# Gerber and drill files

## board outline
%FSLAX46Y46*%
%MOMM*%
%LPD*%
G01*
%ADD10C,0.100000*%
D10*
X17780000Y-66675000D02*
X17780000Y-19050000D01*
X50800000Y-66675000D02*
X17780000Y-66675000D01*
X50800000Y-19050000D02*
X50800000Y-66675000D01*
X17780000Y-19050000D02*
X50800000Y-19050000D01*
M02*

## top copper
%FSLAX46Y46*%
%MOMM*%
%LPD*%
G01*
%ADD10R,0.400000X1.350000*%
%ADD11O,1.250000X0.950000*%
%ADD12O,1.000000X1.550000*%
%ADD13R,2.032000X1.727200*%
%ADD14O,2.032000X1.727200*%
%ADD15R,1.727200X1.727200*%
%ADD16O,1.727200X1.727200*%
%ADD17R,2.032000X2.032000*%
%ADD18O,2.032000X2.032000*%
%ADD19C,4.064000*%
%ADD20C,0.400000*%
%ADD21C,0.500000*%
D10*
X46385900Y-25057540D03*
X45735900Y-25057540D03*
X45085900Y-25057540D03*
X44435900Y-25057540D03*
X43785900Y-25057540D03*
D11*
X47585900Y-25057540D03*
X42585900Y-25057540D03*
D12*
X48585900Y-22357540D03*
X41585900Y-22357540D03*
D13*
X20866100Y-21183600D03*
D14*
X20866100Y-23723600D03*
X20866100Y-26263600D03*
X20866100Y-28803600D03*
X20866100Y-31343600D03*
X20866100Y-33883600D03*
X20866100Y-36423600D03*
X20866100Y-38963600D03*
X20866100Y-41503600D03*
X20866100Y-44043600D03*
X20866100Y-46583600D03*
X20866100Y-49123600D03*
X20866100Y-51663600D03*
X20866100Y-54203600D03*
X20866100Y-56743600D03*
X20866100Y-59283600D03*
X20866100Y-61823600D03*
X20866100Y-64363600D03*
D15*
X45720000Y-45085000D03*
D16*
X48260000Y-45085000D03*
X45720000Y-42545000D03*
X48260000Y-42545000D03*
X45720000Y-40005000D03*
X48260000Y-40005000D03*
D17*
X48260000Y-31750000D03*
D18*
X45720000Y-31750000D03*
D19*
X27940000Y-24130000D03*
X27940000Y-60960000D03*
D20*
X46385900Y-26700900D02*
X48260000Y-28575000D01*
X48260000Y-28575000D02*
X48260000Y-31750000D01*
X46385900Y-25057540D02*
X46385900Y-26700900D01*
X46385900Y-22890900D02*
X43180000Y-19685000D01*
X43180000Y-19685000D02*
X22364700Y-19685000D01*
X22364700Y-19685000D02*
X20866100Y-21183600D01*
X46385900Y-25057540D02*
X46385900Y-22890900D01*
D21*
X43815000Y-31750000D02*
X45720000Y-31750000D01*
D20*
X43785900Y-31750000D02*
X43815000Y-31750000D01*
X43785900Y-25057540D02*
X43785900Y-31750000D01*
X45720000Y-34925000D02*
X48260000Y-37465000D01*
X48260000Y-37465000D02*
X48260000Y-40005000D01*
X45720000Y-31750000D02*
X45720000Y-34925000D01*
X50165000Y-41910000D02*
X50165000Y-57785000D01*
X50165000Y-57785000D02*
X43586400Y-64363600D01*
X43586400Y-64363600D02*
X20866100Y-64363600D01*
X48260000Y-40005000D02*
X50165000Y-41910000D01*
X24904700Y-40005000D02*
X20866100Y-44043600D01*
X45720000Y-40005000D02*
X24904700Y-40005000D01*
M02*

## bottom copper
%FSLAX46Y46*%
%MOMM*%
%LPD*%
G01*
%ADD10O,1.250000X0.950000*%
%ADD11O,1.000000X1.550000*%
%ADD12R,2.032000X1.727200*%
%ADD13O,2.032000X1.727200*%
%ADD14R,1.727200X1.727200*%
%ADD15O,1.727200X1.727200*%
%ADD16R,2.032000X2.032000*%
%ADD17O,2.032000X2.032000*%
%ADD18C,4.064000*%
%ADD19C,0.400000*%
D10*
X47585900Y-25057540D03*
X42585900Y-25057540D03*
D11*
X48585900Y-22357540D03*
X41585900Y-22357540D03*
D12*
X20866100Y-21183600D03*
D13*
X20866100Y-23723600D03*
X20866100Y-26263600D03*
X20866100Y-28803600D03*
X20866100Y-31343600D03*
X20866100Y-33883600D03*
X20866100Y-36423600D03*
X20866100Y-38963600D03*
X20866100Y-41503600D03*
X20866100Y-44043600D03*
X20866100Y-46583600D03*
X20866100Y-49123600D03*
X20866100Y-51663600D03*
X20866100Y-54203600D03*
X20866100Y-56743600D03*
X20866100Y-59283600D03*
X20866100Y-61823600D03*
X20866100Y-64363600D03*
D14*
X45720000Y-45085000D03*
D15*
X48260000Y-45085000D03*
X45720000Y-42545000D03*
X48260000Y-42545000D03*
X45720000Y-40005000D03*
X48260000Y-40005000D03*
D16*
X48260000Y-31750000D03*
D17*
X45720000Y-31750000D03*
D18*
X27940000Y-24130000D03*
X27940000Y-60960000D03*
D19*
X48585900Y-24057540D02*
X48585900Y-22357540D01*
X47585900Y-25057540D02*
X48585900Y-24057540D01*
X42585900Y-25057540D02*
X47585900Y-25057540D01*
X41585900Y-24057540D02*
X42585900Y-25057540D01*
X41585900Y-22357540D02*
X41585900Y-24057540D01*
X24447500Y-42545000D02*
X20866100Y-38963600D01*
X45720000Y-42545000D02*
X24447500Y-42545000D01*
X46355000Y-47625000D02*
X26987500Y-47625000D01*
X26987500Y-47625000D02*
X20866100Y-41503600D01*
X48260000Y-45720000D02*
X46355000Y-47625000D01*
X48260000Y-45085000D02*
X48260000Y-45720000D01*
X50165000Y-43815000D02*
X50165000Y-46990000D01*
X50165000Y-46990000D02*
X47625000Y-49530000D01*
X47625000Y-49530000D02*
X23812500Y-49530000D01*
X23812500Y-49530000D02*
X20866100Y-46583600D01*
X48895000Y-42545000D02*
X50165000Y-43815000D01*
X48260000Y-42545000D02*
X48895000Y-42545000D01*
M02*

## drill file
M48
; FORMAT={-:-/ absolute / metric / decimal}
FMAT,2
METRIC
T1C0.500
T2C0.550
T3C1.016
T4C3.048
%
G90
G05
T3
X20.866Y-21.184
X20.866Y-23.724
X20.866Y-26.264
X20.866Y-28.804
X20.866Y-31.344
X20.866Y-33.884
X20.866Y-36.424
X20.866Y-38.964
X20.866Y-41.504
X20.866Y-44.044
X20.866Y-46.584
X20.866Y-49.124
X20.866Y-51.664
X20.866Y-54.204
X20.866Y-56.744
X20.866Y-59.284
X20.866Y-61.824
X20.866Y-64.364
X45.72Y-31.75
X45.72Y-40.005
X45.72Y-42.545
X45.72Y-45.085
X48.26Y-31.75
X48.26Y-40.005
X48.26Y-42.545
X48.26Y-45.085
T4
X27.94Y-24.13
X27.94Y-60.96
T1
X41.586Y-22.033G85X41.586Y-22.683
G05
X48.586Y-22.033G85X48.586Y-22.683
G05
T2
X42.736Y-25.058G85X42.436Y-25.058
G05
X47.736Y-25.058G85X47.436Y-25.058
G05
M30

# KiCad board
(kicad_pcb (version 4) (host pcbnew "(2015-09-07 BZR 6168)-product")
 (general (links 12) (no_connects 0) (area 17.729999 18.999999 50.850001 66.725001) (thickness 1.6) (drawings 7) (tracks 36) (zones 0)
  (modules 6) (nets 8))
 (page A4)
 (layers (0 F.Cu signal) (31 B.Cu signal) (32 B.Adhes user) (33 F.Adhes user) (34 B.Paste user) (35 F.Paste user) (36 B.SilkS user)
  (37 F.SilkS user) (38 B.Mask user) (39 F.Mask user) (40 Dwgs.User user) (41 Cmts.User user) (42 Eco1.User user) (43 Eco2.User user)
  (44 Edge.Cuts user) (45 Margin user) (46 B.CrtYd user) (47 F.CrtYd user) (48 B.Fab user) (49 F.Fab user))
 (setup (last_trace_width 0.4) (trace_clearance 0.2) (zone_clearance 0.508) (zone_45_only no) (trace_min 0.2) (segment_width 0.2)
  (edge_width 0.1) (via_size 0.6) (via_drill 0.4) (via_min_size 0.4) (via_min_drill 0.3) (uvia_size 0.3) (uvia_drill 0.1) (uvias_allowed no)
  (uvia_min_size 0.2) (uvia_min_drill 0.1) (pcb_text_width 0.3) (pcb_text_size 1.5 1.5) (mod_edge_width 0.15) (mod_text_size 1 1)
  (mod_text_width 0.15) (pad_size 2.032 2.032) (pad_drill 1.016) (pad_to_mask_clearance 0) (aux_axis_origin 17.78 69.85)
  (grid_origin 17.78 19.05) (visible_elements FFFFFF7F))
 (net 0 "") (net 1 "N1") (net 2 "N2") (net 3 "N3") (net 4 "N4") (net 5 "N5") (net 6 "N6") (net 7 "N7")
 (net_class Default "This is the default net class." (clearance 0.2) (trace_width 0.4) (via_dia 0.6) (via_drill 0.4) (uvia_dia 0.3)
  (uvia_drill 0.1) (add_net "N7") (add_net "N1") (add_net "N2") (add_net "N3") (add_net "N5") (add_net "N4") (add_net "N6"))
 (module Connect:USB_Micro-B (layer F.Cu) (at 45.085 23.495 180)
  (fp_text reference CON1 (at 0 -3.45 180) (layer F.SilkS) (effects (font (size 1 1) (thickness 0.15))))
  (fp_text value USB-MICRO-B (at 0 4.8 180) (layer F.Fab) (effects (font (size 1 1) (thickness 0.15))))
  (pad 1 smd rect (at -1.3009 -1.56254 270) (size 1.35 0.4) (layers F.Cu F.Paste F.Mask) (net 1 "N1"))
  (pad 2 smd rect (at -0.6509 -1.56254 270) (size 1.35 0.4) (layers F.Cu F.Paste F.Mask))
  (pad 3 smd rect (at -0.0009 -1.56254 270) (size 1.35 0.4) (layers F.Cu F.Paste F.Mask))
  (pad 4 smd rect (at 0.6491 -1.56254 270) (size 1.35 0.4) (layers F.Cu F.Paste F.Mask))
  (pad 5 smd rect (at 1.2991 -1.56254 270) (size 1.35 0.4) (layers F.Cu F.Paste F.Mask) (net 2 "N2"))
  (pad 6 thru_hole oval (at -2.5009 -1.56254 270) (size 0.95 1.25) (drill oval 0.55 0.85) (layers *.Cu *.Mask F.SilkS) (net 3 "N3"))
  (pad 6 thru_hole oval (at 2.4991 -1.56254 270) (size 0.95 1.25) (drill oval 0.55 0.85) (layers *.Cu *.Mask F.SilkS) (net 3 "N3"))
  (pad 6 thru_hole oval (at -3.5009 1.13746 270) (size 1.55 1) (drill oval 1.15 0.5) (layers *.Cu *.Mask F.SilkS) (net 3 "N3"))
  (pad 6 thru_hole oval (at 3.4991 1.13746 270) (size 1.55 1) (drill oval 1.15 0.5) (layers *.Cu *.Mask F.SilkS) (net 3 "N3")))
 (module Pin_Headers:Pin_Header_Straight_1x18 (layer F.Cu) (at 20.8661 21.1836)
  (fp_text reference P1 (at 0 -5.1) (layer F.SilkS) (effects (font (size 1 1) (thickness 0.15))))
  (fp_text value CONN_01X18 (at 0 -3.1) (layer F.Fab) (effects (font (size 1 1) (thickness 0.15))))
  (pad 1 thru_hole rect (at 0 0) (size 2.032 1.7272) (drill 1.016) (layers *.Cu *.Mask F.SilkS) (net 1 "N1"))
  (pad 2 thru_hole oval (at 0 2.54) (size 2.032 1.7272) (drill 1.016) (layers *.Cu *.Mask F.SilkS))
  (pad 3 thru_hole oval (at 0 5.08) (size 2.032 1.7272) (drill 1.016) (layers *.Cu *.Mask F.SilkS))
  (pad 4 thru_hole oval (at 0 7.62) (size 2.032 1.7272) (drill 1.016) (layers *.Cu *.Mask F.SilkS))
  (pad 5 thru_hole oval (at 0 10.16) (size 2.032 1.7272) (drill 1.016) (layers *.Cu *.Mask F.SilkS))
  (pad 6 thru_hole oval (at 0 12.7) (size 2.032 1.7272) (drill 1.016) (layers *.Cu *.Mask F.SilkS))
  (pad 7 thru_hole oval (at 0 15.24) (size 2.032 1.7272) (drill 1.016) (layers *.Cu *.Mask F.SilkS))
  (pad 8 thru_hole oval (at 0 17.78) (size 2.032 1.7272) (drill 1.016) (layers *.Cu *.Mask F.SilkS) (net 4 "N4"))
  (pad 9 thru_hole oval (at 0 20.32) (size 2.032 1.7272) (drill 1.016) (layers *.Cu *.Mask F.SilkS) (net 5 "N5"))
  (pad 10 thru_hole oval (at 0 22.86) (size 2.032 1.7272) (drill 1.016) (layers *.Cu *.Mask F.SilkS) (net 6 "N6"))
  (pad 11 thru_hole oval (at 0 25.4) (size 2.032 1.7272) (drill 1.016) (layers *.Cu *.Mask F.SilkS) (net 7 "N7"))
  (pad 12 thru_hole oval (at 0 27.94) (size 2.032 1.7272) (drill 1.016) (layers *.Cu *.Mask F.SilkS))
  (pad 13 thru_hole oval (at 0 30.48) (size 2.032 1.7272) (drill 1.016) (layers *.Cu *.Mask F.SilkS))
  (pad 14 thru_hole oval (at 0 33.02) (size 2.032 1.7272) (drill 1.016) (layers *.Cu *.Mask F.SilkS))
  (pad 15 thru_hole oval (at 0 35.56) (size 2.032 1.7272) (drill 1.016) (layers *.Cu *.Mask F.SilkS))
  (pad 16 thru_hole oval (at 0 38.1) (size 2.032 1.7272) (drill 1.016) (layers *.Cu *.Mask F.SilkS))
  (pad 17 thru_hole oval (at 0 40.64) (size 2.032 1.7272) (drill 1.016) (layers *.Cu *.Mask F.SilkS))
  (pad 18 thru_hole oval (at 0 43.18) (size 2.032 1.7272) (drill 1.016) (layers *.Cu *.Mask F.SilkS) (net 2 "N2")))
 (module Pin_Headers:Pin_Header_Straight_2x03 (layer B.Cu) (at 45.72 45.085)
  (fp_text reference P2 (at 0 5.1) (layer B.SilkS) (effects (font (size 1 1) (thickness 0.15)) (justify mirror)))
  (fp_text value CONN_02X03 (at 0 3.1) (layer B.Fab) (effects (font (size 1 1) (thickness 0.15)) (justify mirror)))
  (pad 1 thru_hole rect (at 0 0) (size 1.7272 1.7272) (drill 1.016) (layers *.Cu *.Mask B.SilkS))
  (pad 2 thru_hole oval (at 2.54 0) (size 1.7272 1.7272) (drill 1.016) (layers *.Cu *.Mask B.SilkS) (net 5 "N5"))
  (pad 3 thru_hole oval (at 0 -2.54) (size 1.7272 1.7272) (drill 1.016) (layers *.Cu *.Mask B.SilkS) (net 4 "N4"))
  (pad 4 thru_hole oval (at 2.54 -2.54) (size 1.7272 1.7272) (drill 1.016) (layers *.Cu *.Mask B.SilkS) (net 7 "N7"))
  (pad 5 thru_hole oval (at 0 -5.08) (size 1.7272 1.7272) (drill 1.016) (layers *.Cu *.Mask B.SilkS) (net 6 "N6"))
  (pad 6 thru_hole oval (at 2.54 -5.08) (size 1.7272 1.7272) (drill 1.016) (layers *.Cu *.Mask B.SilkS) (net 2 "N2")))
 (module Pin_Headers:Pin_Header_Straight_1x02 (layer B.Cu) (at 48.26 31.75 90)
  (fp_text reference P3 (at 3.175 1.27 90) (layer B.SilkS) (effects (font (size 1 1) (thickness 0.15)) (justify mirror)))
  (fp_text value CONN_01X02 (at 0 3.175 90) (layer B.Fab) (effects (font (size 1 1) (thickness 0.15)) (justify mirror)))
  (pad 1 thru_hole rect (at 0 0 90) (size 2.032 2.032) (drill 1.016) (layers *.Cu *.Mask B.SilkS) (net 1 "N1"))
  (pad 2 thru_hole oval (at 0 -2.54 90) (size 2.032 2.032) (drill 1.016) (layers *.Cu *.Mask B.SilkS) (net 2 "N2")))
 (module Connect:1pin (layer F.Cu) (at 27.94 24.13)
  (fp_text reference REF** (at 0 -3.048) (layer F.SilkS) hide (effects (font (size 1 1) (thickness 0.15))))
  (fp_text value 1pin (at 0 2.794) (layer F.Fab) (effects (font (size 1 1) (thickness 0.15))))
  (pad 1 thru_hole circle (at 0 0) (size 4.064 4.064) (drill 3.048) (layers *.Cu *.Mask F.SilkS)))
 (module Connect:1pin (layer F.Cu) (at 27.94 60.96)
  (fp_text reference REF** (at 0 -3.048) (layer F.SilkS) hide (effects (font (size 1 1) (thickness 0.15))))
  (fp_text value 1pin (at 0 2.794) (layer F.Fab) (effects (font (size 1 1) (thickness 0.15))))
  (pad 1 thru_hole circle (at 0 0) (size 4.064 4.064) (drill 3.048) (layers *.Cu *.Mask F.SilkS)))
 (gr_line (start 17.78 66.675) (end 17.78 19.05) (angle 90) (layer Edge.Cuts) (width 0.1))
 (gr_line (start 50.8 66.675) (end 17.78 66.675) (angle 90) (layer Edge.Cuts) (width 0.1))
 (gr_line (start 50.8 19.05) (end 50.8 66.675) (angle 90) (layer Edge.Cuts) (width 0.1))
 (gr_line (start 17.78 19.05) (end 50.8 19.05) (angle 90) (layer Edge.Cuts) (width 0.1))
 (segment (start 46.3859 26.7009) (end 48.26 28.575) (width 0.4) (layer F.Cu) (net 1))
 (segment (start 48.26 28.575) (end 48.26 31.75) (width 0.4) (layer F.Cu) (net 1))
 (segment (start 46.3859 25.05754) (end 46.3859 26.7009) (width 0.4) (layer F.Cu) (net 1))
 (segment (start 46.3859 22.8909) (end 43.18 19.685) (width 0.4) (layer F.Cu) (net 1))
 (segment (start 43.18 19.685) (end 22.3647 19.685) (width 0.4) (layer F.Cu) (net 1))
 (segment (start 22.3647 19.685) (end 20.8661 21.1836) (width 0.4) (layer F.Cu) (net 1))
 (segment (start 46.3859 25.05754) (end 46.3859 22.8909) (width 0.4) (layer F.Cu) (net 1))
 (segment (start 43.815 31.75) (end 45.72 31.75) (width 0.5) (layer F.Cu) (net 2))
 (segment (start 43.7859 31.75) (end 43.815 31.75) (width 0.4) (layer F.Cu) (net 2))
 (segment (start 43.7859 25.05754) (end 43.7859 31.75) (width 0.4) (layer F.Cu) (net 2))
 (segment (start 45.72 34.925) (end 48.26 37.465) (width 0.4) (layer F.Cu) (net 2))
 (segment (start 48.26 37.465) (end 48.26 40.005) (width 0.4) (layer F.Cu) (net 2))
 (segment (start 45.72 31.75) (end 45.72 34.925) (width 0.4) (layer F.Cu) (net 2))
 (segment (start 50.165 41.91) (end 50.165 57.785) (width 0.4) (layer F.Cu) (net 2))
 (segment (start 50.165 57.785) (end 43.5864 64.3636) (width 0.4) (layer F.Cu) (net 2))
 (segment (start 43.5864 64.3636) (end 20.8661 64.3636) (width 0.4) (layer F.Cu) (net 2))
 (segment (start 48.26 40.005) (end 50.165 41.91) (width 0.4) (layer F.Cu) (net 2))
 (segment (start 48.5859 24.05754) (end 48.5859 22.35754) (width 0.4) (layer B.Cu) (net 3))
 (segment (start 47.5859 25.05754) (end 48.5859 24.05754) (width 0.4) (layer B.Cu) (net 3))
 (segment (start 42.5859 25.05754) (end 47.5859 25.05754) (width 0.4) (layer B.Cu) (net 3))
 (segment (start 41.5859 24.05754) (end 42.5859 25.05754) (width 0.4) (layer B.Cu) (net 3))
 (segment (start 41.5859 22.35754) (end 41.5859 24.05754) (width 0.4) (layer B.Cu) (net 3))
 (segment (start 24.4475 42.545) (end 20.8661 38.9636) (width 0.4) (layer B.Cu) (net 4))
 (segment (start 45.72 42.545) (end 24.4475 42.545) (width 0.4) (layer B.Cu) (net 4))
 (segment (start 46.355 47.625) (end 26.9875 47.625) (width 0.4) (layer B.Cu) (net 5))
 (segment (start 26.9875 47.625) (end 20.8661 41.5036) (width 0.4) (layer B.Cu) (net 5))
 (segment (start 48.26 45.72) (end 46.355 47.625) (width 0.4) (layer B.Cu) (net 5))
 (segment (start 48.26 45.085) (end 48.26 45.72) (width 0.4) (layer B.Cu) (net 5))
 (segment (start 24.9047 40.005) (end 20.8661 44.0436) (width 0.4) (layer F.Cu) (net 6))
 (segment (start 45.72 40.005) (end 24.9047 40.005) (width 0.4) (layer F.Cu) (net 6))
 (segment (start 50.165 43.815) (end 50.165 46.99) (width 0.4) (layer B.Cu) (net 7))
 (segment (start 50.165 46.99) (end 47.625 49.53) (width 0.4) (layer B.Cu) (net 7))
 (segment (start 47.625 49.53) (end 23.8125 49.53) (width 0.4) (layer B.Cu) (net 7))
 (segment (start 23.8125 49.53) (end 20.8661 46.5836) (width 0.4) (layer B.Cu) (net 7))
 (segment (start 48.895 42.545) (end 50.165 43.815) (width 0.4) (layer B.Cu) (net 7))
 (segment (start 48.26 42.545) (end 48.895 42.545) (width 0.4) (layer B.Cu) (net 7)))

